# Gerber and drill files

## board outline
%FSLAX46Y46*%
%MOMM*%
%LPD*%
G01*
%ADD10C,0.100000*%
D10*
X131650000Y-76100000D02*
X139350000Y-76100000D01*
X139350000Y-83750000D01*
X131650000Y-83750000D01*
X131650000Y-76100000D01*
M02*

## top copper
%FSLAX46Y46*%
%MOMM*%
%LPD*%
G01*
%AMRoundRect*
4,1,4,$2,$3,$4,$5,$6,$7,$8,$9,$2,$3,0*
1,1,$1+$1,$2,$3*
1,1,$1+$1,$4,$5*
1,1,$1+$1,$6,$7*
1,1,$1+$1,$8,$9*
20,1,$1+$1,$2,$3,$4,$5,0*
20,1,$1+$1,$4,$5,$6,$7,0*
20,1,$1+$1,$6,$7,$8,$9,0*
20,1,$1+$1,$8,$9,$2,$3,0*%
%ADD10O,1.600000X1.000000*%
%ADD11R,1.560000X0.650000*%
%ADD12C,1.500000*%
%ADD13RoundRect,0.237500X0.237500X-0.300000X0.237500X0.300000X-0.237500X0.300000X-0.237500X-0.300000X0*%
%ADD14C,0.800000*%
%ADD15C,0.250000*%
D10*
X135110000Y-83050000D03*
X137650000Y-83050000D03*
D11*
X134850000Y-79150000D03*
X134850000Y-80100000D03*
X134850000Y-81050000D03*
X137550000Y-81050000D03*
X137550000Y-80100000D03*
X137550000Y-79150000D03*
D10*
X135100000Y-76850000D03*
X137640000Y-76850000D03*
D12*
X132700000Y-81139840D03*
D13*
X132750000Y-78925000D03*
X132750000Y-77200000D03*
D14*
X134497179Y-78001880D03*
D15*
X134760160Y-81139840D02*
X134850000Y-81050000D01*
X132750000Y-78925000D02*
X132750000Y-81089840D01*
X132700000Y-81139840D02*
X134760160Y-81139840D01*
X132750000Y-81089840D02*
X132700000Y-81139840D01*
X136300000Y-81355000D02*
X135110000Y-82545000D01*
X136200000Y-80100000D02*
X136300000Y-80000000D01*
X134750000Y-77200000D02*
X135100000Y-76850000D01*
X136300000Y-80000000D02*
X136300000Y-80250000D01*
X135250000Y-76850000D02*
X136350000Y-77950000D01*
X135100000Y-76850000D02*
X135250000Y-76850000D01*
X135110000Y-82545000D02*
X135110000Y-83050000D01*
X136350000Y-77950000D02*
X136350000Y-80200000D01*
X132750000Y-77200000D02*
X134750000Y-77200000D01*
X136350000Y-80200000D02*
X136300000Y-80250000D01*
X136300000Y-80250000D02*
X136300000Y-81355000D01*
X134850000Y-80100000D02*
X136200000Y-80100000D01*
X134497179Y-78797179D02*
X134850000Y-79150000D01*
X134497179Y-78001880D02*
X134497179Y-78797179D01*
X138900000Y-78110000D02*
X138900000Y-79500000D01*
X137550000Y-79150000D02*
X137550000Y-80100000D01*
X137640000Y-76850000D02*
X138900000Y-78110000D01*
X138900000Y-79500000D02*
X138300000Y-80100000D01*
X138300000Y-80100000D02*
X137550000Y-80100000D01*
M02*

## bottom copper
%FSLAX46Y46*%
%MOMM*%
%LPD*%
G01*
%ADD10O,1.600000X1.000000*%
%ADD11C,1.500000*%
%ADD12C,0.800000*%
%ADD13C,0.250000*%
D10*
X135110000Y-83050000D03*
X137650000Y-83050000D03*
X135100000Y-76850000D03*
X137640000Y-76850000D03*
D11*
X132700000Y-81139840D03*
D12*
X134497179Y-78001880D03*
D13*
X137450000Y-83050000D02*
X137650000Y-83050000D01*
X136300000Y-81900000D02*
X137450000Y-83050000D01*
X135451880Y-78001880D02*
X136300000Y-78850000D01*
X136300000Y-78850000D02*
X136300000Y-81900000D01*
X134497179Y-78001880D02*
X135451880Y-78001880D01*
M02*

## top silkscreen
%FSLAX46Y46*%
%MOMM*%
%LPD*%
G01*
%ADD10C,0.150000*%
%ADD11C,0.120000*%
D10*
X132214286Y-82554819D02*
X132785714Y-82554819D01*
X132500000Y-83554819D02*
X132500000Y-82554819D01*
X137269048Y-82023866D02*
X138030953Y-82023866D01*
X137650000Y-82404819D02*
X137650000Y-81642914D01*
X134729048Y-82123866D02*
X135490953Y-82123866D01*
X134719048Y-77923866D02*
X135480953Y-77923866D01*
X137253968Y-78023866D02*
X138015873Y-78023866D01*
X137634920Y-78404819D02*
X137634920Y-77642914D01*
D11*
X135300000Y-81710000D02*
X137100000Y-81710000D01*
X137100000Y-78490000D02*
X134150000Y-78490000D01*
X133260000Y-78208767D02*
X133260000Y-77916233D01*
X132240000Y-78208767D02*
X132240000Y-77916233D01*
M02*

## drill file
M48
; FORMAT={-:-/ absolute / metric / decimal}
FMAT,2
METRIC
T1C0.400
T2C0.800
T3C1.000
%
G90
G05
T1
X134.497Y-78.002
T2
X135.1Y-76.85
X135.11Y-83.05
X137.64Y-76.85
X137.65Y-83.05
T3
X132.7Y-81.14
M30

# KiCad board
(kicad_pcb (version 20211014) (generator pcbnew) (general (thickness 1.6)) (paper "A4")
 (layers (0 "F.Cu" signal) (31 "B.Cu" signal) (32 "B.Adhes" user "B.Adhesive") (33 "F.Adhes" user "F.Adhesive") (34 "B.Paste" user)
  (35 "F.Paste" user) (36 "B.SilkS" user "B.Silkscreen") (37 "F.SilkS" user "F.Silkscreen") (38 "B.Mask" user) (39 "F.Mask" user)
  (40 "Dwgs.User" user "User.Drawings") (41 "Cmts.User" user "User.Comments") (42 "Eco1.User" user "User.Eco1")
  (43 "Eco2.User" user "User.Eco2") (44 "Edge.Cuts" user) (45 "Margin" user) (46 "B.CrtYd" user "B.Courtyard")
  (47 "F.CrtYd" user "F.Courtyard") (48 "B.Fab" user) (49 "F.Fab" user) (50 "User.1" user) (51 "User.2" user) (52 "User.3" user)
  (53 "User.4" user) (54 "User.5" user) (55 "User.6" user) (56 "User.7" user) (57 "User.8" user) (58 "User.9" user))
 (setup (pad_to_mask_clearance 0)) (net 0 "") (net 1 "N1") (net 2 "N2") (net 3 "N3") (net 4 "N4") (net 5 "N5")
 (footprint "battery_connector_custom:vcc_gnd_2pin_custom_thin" (layer "F.Cu") (at 136.38 83.05)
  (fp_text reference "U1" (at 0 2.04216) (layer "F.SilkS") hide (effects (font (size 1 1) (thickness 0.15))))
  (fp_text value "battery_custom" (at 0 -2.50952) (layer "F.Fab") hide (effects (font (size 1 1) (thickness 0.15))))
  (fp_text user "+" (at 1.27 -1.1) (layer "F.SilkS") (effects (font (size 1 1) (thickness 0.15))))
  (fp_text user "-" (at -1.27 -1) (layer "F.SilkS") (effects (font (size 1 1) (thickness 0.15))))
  (pad "1" thru_hole oval (at -1.27 0) (size 1.6 1) (drill 0.8) (layers *.Cu *.Mask) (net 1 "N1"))
  (pad "2" thru_hole oval (at 1.27 0) (size 1.6 1) (drill 0.8) (layers *.Cu *.Mask) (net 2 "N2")))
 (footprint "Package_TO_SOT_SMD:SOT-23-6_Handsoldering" (layer "F.Cu") (at 136.2 80.1)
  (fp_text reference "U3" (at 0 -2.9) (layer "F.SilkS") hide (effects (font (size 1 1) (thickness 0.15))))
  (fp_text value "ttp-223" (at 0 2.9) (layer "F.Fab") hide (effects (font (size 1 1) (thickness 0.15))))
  (fp_line (start -0.9 1.61) (end 0.9 1.61) (layer "F.SilkS") (width 0.12))
  (fp_line (start 0.9 -1.61) (end -2.05 -1.61) (layer "F.SilkS") (width 0.12))
  (pad "1" smd rect (at -1.35 -0.95) (size 1.56 0.65) (layers "F.Cu" "F.Paste" "F.Mask") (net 2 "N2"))
  (pad "2" smd rect (at -1.35 0) (size 1.56 0.65) (layers "F.Cu" "F.Paste" "F.Mask") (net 1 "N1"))
  (pad "3" smd rect (at -1.35 0.95) (size 1.56 0.65) (layers "F.Cu" "F.Paste" "F.Mask") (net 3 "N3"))
  (pad "4" smd rect (at 1.35 0.95) (size 1.56 0.65) (layers "F.Cu" "F.Paste" "F.Mask") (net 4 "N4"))
  (pad "5" smd rect (at 1.35 0) (size 1.56 0.65) (layers "F.Cu" "F.Paste" "F.Mask") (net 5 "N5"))
  (pad "6" smd rect (at 1.35 -0.95) (size 1.56 0.65) (layers "F.Cu" "F.Paste" "F.Mask") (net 5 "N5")))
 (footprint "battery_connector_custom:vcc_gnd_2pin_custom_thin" (layer "F.Cu") (at 136.37 76.85)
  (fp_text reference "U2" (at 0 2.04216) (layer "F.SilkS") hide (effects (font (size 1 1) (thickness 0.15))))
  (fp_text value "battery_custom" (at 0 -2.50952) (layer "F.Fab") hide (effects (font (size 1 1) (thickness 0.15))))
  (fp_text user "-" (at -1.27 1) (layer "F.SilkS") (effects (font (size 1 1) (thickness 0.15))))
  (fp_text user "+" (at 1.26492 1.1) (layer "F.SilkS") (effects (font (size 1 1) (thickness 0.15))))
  (pad "1" thru_hole oval (at -1.27 0) (size 1.6 1) (drill 0.8) (layers *.Cu *.Mask) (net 1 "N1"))
  (pad "2" thru_hole oval (at 1.27 0) (size 1.6 1) (drill 0.8) (layers *.Cu *.Mask) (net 5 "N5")))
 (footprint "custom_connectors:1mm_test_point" (layer "F.Cu") (at 132.7 81.15)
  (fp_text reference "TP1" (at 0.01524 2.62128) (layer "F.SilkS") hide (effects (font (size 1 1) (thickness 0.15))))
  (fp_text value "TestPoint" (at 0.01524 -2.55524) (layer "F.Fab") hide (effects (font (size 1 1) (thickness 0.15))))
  (pad "1" thru_hole circle locked (at 0 -0.01016) (size 1.5 1.5) (drill 1) (layers *.Cu *.Mask) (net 3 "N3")))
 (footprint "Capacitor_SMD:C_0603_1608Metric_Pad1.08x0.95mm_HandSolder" (layer "F.Cu") (at 132.75 78.0625 90)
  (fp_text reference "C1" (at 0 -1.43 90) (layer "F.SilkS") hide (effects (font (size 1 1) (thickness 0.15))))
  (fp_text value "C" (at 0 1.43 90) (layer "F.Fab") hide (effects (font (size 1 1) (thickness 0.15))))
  (fp_line (start -0.146267 0.51) (end 0.146267 0.51) (layer "F.SilkS") (width 0.12))
  (fp_line (start -0.146267 -0.51) (end 0.146267 -0.51) (layer "F.SilkS") (width 0.12))
  (pad "1" smd roundrect (at -0.8625 0 90) (size 1.075 0.95) (layers "F.Cu" "F.Paste" "F.Mask") (roundrect_rratio 0.25) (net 3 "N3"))
  (pad "2" smd roundrect (at 0.8625 0 90) (size 1.075 0.95) (layers "F.Cu" "F.Paste" "F.Mask") (roundrect_rratio 0.25) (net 1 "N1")))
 (gr_rect (start 131.65 76.1) (end 139.35 83.75) (layer "Edge.Cuts") (width 0.1) (fill none))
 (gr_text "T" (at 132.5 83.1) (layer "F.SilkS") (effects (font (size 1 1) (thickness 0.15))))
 (segment (start 134.76016 81.13984) (end 134.85 81.05) (width 0.25) (layer "F.Cu") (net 3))
 (segment (start 132.75 78.925) (end 132.75 81.08984) (width 0.25) (layer "F.Cu") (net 3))
 (segment (start 132.7 81.13984) (end 134.76016 81.13984) (width 0.25) (layer "F.Cu") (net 3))
 (segment (start 132.75 81.08984) (end 132.7 81.13984) (width 0.25) (layer "F.Cu") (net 3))
 (segment (start 136.3 81.355) (end 135.11 82.545) (width 0.25) (layer "F.Cu") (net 1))
 (segment (start 136.2 80.1) (end 136.3 80) (width 0.25) (layer "F.Cu") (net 1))
 (segment (start 134.75 77.2) (end 135.1 76.85) (width 0.25) (layer "F.Cu") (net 1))
 (segment (start 136.3 80) (end 136.3 80.25) (width 0.25) (layer "F.Cu") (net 1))
 (segment (start 135.25 76.85) (end 136.35 77.95) (width 0.25) (layer "F.Cu") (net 1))
 (segment (start 135.1 76.85) (end 135.25 76.85) (width 0.25) (layer "F.Cu") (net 1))
 (segment (start 135.11 82.545) (end 135.11 83.05) (width 0.25) (layer "F.Cu") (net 1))
 (segment (start 136.35 77.95) (end 136.35 80.2) (width 0.25) (layer "F.Cu") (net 1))
 (segment (start 132.75 77.2) (end 134.75 77.2) (width 0.25) (layer "F.Cu") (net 1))
 (segment (start 136.35 80.2) (end 136.3 80.25) (width 0.25) (layer "F.Cu") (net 1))
 (segment (start 136.3 80.25) (end 136.3 81.355) (width 0.25) (layer "F.Cu") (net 1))
 (segment (start 134.85 80.1) (end 136.2 80.1) (width 0.25) (layer "F.Cu") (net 1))
 (segment (start 134.497179 78.797179) (end 134.85 79.15) (width 0.25) (layer "F.Cu") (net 2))
 (segment (start 134.497179 78.00188) (end 134.497179 78.797179) (width 0.25) (layer "F.Cu") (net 2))
 (via (at 134.497179 78.00188) (size 0.8) (drill 0.4) (layers "F.Cu" "B.Cu") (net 2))
 (segment (start 137.45 83.05) (end 137.65 83.05) (width 0.25) (layer "B.Cu") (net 2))
 (segment (start 136.3 81.9) (end 137.45 83.05) (width 0.25) (layer "B.Cu") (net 2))
 (segment (start 135.45188 78.00188) (end 136.3 78.85) (width 0.25) (layer "B.Cu") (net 2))
 (segment (start 136.3 78.85) (end 136.3 81.9) (width 0.25) (layer "B.Cu") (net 2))
 (segment (start 134.497179 78.00188) (end 135.45188 78.00188) (width 0.25) (layer "B.Cu") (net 2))
 (segment (start 138.9 78.11) (end 138.9 79.5) (width 0.25) (layer "F.Cu") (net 5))
 (segment (start 137.55 79.15) (end 137.55 80.1) (width 0.25) (layer "F.Cu") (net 5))
 (segment (start 137.64 76.85) (end 138.9 78.11) (width 0.25) (layer "F.Cu") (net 5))
 (segment (start 138.9 79.5) (end 138.3 80.1) (width 0.25) (layer "F.Cu") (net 5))
 (segment (start 138.3 80.1) (end 137.55 80.1) (width 0.25) (layer "F.Cu") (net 5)))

